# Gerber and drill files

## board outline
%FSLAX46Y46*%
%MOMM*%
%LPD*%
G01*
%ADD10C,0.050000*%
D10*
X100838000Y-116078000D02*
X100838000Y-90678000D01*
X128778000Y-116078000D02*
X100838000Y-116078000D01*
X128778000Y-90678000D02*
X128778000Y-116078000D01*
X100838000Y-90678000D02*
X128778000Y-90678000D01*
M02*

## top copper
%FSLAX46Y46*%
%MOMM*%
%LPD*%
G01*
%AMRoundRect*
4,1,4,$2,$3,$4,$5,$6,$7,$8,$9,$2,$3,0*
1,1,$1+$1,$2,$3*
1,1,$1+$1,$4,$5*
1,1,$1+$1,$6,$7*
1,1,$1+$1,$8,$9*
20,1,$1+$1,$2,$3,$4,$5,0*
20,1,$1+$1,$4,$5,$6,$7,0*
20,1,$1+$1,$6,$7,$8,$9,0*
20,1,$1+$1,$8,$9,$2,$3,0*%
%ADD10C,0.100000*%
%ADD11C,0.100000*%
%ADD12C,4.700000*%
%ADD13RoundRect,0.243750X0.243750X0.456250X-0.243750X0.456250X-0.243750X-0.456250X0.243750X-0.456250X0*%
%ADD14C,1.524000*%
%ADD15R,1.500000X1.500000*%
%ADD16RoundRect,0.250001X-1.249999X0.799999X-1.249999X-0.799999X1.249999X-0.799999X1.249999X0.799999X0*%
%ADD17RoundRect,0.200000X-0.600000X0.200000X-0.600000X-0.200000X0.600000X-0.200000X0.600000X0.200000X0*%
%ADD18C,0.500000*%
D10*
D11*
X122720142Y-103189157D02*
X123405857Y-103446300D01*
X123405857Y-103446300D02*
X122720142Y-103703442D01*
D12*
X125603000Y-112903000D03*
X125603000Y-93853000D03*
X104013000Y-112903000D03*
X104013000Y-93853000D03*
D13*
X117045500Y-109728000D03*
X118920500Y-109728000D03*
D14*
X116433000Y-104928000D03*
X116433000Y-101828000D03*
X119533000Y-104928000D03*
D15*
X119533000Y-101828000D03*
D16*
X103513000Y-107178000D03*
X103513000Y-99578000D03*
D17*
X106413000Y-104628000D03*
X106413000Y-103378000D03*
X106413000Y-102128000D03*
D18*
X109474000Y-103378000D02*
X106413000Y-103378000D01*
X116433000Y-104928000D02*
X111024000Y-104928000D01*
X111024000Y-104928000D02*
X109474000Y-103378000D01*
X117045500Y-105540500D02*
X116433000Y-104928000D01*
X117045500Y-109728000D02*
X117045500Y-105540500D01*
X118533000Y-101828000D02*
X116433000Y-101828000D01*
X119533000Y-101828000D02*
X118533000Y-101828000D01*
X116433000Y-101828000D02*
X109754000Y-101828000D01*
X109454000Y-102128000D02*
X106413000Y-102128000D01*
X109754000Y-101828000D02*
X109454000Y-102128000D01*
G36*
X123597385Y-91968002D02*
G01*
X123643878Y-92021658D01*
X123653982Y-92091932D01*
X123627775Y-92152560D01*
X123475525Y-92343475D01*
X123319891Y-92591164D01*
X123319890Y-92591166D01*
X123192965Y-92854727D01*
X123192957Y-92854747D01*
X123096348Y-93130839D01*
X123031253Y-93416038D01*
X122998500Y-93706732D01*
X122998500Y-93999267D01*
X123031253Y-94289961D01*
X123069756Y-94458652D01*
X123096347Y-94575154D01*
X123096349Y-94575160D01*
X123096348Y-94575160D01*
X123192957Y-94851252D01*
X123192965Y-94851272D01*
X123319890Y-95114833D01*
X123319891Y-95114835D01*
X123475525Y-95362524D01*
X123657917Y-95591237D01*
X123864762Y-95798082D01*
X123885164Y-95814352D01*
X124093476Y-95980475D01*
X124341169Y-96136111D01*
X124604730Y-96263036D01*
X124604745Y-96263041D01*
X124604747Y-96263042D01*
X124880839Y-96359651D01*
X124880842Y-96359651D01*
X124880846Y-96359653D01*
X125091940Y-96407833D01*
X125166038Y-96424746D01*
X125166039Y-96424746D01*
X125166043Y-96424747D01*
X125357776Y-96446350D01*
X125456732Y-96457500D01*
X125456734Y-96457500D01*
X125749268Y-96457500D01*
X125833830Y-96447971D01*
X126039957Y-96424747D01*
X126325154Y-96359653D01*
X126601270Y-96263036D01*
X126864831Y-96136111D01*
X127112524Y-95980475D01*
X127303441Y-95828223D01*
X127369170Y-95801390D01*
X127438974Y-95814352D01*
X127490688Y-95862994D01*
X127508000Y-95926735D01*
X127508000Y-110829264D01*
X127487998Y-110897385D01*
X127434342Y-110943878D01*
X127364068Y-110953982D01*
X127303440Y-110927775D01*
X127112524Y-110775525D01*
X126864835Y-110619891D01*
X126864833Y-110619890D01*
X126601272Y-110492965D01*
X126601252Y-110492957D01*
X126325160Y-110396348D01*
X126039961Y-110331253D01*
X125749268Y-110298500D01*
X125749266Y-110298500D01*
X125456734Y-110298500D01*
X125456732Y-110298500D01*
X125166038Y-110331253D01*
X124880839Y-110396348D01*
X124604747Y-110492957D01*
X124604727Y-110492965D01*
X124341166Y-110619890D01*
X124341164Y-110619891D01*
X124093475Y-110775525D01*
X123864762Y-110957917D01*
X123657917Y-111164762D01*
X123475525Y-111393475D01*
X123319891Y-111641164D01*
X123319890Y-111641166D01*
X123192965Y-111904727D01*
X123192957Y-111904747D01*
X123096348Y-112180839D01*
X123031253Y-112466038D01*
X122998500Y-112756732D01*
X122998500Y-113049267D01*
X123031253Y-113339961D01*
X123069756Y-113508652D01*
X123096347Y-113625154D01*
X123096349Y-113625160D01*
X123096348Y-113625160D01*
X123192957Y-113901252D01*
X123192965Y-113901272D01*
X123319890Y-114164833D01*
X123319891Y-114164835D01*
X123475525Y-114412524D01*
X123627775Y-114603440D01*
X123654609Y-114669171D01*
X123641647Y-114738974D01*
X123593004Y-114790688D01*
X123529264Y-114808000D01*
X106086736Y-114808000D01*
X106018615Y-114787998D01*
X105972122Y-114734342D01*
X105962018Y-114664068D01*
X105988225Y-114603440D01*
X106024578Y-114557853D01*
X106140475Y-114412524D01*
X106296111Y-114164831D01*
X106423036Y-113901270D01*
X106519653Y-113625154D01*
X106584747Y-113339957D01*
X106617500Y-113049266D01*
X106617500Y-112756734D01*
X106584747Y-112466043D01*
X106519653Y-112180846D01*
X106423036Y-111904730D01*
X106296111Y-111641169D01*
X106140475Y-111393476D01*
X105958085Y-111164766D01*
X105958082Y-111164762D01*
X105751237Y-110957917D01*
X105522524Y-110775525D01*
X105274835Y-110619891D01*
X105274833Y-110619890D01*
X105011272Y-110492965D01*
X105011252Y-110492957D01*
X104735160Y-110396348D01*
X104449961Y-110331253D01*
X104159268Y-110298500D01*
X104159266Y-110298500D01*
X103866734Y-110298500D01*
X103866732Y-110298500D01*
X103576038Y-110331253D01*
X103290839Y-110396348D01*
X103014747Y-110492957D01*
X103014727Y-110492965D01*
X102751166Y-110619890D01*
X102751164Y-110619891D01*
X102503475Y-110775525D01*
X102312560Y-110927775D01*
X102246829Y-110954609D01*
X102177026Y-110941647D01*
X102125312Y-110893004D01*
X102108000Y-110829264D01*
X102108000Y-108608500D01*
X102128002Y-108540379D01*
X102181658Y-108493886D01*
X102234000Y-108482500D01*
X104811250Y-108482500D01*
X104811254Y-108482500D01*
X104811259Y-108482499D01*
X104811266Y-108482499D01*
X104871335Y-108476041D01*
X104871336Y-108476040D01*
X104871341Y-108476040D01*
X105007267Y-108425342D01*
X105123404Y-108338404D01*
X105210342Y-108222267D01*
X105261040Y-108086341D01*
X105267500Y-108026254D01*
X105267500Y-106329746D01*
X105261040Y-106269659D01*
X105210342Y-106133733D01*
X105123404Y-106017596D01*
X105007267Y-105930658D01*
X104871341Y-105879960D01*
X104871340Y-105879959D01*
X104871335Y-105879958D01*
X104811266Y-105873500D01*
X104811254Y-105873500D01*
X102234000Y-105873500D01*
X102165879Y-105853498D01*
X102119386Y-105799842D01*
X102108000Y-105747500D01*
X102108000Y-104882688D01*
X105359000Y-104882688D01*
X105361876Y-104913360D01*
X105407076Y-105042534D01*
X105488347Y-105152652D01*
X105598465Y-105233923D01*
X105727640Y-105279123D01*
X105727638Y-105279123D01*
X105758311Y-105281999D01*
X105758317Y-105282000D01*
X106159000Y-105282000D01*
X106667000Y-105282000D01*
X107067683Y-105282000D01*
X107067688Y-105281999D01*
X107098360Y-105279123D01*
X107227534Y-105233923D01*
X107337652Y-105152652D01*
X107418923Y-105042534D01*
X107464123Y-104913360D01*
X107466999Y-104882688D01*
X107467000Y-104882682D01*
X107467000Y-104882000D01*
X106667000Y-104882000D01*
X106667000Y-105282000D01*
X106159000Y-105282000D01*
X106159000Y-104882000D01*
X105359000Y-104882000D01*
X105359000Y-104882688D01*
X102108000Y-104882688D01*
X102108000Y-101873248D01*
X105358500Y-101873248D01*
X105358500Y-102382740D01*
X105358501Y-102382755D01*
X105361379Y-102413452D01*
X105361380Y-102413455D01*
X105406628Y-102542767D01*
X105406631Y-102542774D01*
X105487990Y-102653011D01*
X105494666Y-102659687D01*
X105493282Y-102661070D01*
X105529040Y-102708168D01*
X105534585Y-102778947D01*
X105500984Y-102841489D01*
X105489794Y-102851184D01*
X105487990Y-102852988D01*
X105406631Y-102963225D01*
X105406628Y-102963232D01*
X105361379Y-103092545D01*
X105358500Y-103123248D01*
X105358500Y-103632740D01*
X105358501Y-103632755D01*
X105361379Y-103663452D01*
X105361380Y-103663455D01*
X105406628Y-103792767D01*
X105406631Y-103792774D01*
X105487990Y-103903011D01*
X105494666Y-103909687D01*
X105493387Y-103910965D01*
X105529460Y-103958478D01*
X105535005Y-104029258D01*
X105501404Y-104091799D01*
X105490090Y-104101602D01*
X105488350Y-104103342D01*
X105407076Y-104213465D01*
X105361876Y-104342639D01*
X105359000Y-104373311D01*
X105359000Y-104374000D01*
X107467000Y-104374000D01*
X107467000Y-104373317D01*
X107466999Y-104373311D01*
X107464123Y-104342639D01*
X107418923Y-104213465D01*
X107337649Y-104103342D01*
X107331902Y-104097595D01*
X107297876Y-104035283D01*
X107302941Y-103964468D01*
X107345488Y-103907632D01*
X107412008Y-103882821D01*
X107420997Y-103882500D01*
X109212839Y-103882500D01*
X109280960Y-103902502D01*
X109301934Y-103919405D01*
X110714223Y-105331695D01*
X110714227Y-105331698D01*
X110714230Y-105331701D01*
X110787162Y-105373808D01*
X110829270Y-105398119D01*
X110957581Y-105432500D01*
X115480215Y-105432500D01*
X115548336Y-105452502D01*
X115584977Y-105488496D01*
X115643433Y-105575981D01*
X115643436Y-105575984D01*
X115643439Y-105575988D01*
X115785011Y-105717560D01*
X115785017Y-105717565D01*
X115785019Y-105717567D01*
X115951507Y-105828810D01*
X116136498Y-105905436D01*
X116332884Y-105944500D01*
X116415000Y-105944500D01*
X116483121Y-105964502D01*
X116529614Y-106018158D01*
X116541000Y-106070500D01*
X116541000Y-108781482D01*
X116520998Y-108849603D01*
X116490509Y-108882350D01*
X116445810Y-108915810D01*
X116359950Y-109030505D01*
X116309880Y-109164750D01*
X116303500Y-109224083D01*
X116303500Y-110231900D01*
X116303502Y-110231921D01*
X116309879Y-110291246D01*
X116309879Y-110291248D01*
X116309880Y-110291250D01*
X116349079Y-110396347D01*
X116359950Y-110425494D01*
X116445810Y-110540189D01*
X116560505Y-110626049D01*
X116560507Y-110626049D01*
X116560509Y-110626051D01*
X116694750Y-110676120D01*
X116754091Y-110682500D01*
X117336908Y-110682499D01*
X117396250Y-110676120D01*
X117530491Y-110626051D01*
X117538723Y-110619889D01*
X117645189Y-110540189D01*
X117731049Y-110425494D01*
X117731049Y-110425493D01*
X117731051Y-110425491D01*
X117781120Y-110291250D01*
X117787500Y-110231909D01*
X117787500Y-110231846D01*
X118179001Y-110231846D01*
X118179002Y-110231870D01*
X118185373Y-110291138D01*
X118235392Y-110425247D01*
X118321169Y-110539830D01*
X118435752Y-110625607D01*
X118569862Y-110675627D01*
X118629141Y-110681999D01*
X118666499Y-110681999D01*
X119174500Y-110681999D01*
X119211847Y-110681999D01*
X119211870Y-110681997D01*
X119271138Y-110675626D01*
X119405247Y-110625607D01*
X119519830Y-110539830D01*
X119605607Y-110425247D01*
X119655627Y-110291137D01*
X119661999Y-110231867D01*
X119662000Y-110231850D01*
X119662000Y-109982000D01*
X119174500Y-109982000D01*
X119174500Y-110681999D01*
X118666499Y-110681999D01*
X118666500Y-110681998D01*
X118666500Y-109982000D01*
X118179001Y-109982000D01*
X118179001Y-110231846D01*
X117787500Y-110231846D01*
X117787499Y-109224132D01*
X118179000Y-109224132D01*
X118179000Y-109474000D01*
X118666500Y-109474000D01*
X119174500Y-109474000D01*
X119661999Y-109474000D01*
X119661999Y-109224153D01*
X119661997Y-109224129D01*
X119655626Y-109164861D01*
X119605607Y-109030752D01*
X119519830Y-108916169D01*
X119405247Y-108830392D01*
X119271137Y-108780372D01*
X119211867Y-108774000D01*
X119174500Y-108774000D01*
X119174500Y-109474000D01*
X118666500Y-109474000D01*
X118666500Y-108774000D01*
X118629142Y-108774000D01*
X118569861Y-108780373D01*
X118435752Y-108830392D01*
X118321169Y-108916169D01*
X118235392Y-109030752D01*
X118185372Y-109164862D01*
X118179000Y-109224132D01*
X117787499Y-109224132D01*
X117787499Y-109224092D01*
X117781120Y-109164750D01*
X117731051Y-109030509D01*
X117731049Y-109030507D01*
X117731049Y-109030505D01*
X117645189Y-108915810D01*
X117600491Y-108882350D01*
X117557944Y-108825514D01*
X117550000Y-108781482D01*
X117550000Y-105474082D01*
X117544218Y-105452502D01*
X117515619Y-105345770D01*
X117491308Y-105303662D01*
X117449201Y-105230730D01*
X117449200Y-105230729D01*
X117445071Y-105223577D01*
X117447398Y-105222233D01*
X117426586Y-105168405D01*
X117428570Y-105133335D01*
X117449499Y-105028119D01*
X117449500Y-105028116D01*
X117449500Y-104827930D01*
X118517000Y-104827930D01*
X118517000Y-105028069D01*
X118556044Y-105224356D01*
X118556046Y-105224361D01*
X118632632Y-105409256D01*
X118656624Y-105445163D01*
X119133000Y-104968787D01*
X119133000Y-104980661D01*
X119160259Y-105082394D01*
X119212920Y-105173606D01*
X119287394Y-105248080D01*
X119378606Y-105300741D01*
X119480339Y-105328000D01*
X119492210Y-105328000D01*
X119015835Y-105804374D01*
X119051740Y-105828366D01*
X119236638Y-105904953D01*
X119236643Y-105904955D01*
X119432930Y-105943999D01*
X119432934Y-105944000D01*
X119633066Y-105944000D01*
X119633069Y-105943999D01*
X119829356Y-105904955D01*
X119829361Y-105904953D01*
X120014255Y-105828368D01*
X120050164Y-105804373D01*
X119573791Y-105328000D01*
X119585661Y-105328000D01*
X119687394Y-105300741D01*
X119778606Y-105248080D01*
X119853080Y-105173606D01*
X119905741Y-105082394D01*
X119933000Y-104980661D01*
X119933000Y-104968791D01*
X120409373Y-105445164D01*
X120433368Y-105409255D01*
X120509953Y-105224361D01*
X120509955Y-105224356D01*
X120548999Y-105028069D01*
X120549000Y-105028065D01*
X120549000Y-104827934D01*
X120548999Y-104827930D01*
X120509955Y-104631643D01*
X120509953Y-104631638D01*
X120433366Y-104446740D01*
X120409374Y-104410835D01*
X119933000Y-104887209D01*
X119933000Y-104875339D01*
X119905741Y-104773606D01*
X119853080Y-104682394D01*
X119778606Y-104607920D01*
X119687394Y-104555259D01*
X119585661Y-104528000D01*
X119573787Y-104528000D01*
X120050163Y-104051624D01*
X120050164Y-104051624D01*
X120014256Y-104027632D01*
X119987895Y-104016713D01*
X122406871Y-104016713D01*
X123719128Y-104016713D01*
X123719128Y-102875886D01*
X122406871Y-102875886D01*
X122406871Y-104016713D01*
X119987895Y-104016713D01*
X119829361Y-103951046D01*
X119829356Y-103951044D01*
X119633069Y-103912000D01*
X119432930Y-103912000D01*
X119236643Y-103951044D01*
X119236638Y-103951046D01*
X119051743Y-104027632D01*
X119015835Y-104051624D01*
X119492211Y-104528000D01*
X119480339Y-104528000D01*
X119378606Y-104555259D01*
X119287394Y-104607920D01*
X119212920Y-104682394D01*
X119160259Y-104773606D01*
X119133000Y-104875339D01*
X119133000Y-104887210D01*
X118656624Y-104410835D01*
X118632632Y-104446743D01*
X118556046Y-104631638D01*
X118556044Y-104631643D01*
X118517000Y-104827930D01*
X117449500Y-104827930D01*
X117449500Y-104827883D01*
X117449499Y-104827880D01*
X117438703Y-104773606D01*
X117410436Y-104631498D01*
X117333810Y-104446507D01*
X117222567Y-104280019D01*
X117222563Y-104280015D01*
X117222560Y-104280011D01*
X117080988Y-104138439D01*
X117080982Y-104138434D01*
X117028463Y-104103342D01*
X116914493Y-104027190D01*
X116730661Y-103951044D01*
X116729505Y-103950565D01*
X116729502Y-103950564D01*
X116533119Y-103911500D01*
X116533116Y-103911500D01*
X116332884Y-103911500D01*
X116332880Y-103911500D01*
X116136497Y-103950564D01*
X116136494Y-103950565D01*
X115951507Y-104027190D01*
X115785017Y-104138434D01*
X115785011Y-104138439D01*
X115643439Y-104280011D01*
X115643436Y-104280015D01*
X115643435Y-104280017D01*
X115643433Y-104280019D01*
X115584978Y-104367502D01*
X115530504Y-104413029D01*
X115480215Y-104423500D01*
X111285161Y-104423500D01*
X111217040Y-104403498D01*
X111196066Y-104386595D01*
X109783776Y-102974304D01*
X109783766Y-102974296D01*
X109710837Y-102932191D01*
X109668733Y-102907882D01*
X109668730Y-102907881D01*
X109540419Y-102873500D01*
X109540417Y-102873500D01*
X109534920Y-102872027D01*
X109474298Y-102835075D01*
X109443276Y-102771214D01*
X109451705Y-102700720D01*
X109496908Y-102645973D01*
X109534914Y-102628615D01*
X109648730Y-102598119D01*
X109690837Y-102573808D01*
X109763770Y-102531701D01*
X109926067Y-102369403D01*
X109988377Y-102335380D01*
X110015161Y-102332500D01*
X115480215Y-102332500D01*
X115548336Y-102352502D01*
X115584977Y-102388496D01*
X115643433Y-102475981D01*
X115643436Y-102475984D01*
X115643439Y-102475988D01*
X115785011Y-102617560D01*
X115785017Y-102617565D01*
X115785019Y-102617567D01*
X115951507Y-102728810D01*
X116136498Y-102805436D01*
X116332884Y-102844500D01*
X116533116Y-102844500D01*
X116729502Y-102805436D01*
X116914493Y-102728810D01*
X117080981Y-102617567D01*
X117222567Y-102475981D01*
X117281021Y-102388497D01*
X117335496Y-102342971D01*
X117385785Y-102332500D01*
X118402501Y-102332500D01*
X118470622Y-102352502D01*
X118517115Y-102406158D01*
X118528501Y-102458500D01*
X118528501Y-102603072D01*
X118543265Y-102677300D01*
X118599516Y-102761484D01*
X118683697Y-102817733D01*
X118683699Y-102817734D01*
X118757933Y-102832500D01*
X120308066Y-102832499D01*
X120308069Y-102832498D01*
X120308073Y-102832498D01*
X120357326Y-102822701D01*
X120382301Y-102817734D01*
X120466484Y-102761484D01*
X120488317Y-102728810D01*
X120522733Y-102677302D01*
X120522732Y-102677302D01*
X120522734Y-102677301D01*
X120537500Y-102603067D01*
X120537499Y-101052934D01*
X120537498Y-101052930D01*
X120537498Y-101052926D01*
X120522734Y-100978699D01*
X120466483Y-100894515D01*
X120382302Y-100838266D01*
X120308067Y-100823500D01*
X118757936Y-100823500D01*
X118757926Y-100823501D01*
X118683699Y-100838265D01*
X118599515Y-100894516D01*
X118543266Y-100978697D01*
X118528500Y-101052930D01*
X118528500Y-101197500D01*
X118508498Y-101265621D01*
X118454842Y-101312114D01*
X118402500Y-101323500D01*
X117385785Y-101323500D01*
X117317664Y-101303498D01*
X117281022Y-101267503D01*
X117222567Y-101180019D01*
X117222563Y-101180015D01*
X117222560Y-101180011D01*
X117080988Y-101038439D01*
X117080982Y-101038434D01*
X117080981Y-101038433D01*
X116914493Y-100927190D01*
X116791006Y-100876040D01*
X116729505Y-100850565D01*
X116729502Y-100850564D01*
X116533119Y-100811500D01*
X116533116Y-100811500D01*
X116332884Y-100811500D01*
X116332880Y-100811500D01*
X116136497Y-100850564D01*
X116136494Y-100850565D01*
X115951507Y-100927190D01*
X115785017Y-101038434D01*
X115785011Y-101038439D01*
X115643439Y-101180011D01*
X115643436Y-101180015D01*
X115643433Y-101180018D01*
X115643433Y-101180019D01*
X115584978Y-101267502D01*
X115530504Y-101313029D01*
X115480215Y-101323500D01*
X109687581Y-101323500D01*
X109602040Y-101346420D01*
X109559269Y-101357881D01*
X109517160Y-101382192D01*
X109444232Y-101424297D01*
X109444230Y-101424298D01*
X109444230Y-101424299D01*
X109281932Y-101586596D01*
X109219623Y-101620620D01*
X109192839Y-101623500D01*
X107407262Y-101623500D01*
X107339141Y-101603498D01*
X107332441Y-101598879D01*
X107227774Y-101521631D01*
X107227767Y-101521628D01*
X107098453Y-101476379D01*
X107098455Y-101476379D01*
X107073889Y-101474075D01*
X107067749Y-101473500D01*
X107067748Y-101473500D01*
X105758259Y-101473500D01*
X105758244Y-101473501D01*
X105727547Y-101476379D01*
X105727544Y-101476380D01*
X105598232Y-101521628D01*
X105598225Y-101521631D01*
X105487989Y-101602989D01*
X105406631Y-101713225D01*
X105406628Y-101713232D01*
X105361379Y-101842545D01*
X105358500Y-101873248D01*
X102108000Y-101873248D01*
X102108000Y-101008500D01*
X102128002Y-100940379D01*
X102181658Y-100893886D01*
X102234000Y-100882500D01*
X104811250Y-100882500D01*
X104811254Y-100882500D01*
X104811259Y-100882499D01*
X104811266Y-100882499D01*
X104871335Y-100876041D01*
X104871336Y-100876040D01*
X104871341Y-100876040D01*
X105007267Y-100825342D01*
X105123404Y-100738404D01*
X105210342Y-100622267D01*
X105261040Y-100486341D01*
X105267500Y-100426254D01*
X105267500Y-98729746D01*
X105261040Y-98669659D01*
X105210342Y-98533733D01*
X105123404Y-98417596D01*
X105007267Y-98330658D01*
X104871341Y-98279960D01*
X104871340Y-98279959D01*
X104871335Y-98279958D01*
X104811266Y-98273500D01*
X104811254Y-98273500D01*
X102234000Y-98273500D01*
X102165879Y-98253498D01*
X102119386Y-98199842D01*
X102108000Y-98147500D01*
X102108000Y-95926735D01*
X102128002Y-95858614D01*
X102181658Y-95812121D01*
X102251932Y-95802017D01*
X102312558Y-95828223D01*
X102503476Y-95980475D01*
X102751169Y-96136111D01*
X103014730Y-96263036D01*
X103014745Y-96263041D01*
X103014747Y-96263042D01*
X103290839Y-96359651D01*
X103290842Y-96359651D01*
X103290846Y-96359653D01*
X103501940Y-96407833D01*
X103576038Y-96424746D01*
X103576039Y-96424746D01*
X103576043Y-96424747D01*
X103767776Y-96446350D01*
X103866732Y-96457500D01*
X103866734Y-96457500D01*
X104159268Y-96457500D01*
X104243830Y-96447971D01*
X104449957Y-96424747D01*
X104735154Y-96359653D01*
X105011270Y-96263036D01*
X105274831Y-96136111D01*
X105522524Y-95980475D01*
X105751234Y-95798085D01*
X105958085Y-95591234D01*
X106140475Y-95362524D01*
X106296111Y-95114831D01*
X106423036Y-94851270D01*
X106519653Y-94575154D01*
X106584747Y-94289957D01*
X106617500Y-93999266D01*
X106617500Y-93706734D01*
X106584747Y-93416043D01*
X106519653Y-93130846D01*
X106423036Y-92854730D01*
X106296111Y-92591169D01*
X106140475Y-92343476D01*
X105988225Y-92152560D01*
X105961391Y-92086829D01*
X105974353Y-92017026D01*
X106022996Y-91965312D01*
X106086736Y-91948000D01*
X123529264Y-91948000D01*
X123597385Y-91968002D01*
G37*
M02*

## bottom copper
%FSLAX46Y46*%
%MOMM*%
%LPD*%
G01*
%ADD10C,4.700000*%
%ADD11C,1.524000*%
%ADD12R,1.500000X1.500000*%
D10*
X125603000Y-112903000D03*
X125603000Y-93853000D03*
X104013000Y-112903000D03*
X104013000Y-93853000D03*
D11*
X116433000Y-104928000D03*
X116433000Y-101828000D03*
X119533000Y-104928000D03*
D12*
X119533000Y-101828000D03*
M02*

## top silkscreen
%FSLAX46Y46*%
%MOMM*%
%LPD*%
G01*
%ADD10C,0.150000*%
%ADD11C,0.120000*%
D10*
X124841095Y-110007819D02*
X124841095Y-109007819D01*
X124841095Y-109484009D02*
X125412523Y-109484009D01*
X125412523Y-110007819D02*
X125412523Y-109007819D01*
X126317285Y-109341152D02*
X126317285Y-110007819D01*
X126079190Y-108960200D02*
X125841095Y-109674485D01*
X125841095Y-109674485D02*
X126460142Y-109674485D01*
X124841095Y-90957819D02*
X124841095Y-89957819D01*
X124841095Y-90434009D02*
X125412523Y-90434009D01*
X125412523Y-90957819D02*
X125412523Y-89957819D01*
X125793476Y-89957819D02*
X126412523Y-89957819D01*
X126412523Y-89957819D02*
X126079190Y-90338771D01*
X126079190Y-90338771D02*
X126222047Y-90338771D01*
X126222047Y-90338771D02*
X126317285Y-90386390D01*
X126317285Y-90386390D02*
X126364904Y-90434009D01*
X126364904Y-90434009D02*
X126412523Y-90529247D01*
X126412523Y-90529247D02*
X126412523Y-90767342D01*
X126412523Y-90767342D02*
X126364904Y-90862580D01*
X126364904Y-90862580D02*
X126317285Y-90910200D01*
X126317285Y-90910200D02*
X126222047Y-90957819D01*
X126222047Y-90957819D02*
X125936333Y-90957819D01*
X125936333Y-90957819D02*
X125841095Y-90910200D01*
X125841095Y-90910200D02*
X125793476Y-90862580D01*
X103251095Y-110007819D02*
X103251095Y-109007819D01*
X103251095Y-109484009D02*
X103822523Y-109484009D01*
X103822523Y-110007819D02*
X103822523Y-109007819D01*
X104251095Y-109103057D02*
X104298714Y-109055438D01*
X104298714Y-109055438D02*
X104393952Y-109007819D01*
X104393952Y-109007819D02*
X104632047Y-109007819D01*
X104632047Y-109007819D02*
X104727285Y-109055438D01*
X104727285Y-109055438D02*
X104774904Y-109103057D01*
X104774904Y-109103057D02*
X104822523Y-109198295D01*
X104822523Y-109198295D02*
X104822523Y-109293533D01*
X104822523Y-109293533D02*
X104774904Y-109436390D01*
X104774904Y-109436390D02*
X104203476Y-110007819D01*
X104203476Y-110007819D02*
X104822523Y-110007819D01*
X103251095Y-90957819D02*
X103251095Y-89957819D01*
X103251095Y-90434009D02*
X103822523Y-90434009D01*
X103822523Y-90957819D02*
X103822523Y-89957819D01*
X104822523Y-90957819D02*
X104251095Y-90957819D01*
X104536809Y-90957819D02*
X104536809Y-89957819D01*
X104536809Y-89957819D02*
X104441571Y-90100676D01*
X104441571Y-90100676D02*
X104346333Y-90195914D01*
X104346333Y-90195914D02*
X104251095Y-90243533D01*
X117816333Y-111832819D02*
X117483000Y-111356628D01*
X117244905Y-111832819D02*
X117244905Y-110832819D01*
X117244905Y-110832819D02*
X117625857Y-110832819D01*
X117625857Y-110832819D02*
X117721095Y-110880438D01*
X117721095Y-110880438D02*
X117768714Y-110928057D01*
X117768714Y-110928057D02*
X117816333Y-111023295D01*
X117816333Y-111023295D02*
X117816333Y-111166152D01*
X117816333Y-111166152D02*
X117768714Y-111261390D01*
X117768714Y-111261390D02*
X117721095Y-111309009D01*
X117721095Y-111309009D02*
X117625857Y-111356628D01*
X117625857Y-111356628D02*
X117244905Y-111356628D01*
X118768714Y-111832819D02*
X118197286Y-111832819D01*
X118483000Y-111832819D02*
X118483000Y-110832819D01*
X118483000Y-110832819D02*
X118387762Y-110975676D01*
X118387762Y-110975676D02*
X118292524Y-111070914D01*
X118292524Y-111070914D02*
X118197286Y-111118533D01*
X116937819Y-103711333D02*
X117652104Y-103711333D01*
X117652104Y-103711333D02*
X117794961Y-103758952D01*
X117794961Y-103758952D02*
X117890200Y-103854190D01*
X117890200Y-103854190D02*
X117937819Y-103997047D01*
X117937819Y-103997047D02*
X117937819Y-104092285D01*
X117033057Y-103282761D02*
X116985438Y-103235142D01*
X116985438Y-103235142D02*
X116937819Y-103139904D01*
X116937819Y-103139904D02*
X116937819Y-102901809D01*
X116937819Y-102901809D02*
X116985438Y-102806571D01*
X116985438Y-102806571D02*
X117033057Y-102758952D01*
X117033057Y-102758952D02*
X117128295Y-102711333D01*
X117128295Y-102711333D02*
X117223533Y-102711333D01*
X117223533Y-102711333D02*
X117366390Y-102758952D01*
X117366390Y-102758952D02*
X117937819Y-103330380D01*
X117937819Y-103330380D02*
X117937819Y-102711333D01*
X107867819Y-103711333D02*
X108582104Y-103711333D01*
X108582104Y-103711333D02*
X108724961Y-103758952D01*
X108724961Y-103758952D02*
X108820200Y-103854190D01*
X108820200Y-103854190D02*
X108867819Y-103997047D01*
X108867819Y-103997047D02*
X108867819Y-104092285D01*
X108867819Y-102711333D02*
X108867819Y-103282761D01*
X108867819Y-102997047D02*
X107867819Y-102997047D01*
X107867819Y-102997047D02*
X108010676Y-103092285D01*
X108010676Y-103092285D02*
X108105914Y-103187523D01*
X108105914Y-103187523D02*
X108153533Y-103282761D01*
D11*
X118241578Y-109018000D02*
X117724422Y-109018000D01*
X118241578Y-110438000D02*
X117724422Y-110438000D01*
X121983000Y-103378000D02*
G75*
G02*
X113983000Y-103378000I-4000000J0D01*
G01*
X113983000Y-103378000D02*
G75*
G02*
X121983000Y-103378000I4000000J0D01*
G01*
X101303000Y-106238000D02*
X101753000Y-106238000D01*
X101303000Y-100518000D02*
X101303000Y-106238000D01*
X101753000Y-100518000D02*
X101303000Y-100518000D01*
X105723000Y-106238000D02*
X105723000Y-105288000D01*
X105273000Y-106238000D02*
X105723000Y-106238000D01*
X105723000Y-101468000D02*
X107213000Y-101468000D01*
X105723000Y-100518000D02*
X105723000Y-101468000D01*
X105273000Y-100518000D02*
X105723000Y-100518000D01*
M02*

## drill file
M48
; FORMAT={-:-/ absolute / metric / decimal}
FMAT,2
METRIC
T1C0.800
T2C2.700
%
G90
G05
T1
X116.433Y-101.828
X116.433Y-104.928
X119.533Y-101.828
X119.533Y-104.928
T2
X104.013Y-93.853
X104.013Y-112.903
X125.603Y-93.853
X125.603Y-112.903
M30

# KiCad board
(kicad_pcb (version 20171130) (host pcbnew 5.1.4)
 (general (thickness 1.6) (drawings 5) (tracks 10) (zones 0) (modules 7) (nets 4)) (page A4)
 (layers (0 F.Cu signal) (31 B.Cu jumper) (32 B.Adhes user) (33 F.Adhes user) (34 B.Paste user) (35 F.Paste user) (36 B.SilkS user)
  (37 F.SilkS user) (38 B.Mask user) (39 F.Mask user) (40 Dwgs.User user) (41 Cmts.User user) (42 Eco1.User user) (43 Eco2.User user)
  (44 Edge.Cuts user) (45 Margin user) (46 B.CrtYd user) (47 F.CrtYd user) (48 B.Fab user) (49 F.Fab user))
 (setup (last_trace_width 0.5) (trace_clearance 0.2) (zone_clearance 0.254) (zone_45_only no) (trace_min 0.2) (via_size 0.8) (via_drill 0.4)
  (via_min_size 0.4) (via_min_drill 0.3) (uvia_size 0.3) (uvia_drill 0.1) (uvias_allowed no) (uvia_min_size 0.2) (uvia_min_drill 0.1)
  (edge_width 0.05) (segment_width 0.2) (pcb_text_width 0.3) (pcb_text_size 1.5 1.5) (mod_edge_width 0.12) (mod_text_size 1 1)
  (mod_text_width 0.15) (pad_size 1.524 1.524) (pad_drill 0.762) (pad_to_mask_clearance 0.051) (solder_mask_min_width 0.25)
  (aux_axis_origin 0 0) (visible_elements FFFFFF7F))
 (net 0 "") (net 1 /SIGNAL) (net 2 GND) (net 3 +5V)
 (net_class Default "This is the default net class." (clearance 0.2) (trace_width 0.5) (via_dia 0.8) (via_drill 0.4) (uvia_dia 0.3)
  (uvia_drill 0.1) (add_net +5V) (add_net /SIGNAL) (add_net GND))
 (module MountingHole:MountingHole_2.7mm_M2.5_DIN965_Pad (layer F.Cu) (at 125.603 112.903)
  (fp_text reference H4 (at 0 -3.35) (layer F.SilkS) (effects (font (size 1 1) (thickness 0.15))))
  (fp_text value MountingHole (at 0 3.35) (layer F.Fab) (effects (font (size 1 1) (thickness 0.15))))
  (pad 1 thru_hole circle (at 0 0) (size 4.7 4.7) (drill 2.7) (layers *.Cu *.Mask)))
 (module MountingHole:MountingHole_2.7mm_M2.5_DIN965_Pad (layer F.Cu) (at 125.603 93.853)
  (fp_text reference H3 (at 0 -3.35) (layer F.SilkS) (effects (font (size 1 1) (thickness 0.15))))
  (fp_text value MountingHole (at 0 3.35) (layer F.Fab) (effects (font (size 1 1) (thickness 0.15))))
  (pad 1 thru_hole circle (at 0 0) (size 4.7 4.7) (drill 2.7) (layers *.Cu *.Mask)))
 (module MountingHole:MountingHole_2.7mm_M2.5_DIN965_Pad (layer F.Cu) (at 104.013 112.903)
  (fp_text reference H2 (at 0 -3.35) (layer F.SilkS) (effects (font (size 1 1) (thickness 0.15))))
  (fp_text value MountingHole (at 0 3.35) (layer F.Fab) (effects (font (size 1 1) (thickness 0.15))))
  (pad 1 thru_hole circle (at 0 0) (size 4.7 4.7) (drill 2.7) (layers *.Cu *.Mask)))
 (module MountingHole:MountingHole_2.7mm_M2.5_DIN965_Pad (layer F.Cu) (at 104.013 93.853)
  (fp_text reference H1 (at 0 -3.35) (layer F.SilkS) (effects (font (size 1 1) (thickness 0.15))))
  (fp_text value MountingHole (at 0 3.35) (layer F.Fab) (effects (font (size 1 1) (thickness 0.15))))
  (pad 1 thru_hole circle (at 0 0) (size 4.7 4.7) (drill 2.7) (layers *.Cu *.Mask)))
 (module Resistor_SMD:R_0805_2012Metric (layer F.Cu) (at 117.983 109.728 180)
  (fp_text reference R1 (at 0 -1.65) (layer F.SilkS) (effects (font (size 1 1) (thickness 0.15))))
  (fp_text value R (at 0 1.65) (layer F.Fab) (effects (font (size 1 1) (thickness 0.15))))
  (fp_line (start -0.258578 0.71) (end 0.258578 0.71) (layer F.SilkS) (width 0.12))
  (fp_line (start -0.258578 -0.71) (end 0.258578 -0.71) (layer F.SilkS) (width 0.12))
  (pad 2 smd roundrect (at 0.9375 0 180) (size 0.975 1.4) (layers F.Cu F.Paste F.Mask) (roundrect_rratio 0.25) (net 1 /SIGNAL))
  (pad 1 smd roundrect (at -0.9375 0 180) (size 0.975 1.4) (layers F.Cu F.Paste F.Mask) (roundrect_rratio 0.25) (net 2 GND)))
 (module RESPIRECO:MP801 (layer F.Cu) (at 117.983 103.378 270)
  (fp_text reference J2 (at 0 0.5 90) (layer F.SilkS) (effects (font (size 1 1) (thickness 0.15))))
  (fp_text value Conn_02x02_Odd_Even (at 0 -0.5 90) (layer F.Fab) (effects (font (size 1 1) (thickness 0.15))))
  (fp_circle (center 0 0) (end 4 0) (layer F.SilkS) (width 0.12))
  (pad 4 thru_hole circle (at 1.55 1.55 270) (size 1.524 1.524) (drill 0.8) (layers *.Cu *.Mask) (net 1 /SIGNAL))
  (pad 3 thru_hole circle (at -1.55 1.55 270) (size 1.524 1.524) (drill 0.8) (layers *.Cu *.Mask) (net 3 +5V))
  (pad 2 thru_hole circle (at 1.55 -1.55 270) (size 1.524 1.524) (drill 0.8) (layers *.Cu *.Mask) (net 2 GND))
  (pad 1 thru_hole rect (at -1.55 -1.55 270) (size 1.5 1.5) (drill 0.8) (layers *.Cu *.Mask) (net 3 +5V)))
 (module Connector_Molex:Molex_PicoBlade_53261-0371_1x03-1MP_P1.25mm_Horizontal (layer F.Cu) (at 104.013 103.378 270)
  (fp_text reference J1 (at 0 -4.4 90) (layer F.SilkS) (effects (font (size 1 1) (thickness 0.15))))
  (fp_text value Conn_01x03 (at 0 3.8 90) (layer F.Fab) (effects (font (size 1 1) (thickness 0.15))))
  (fp_line (start 2.86 2.71) (end 2.86 2.26) (layer F.SilkS) (width 0.12))
  (fp_line (start -2.86 2.71) (end 2.86 2.71) (layer F.SilkS) (width 0.12))
  (fp_line (start -2.86 2.26) (end -2.86 2.71) (layer F.SilkS) (width 0.12))
  (fp_line (start 2.86 -1.71) (end 1.91 -1.71) (layer F.SilkS) (width 0.12))
  (fp_line (start 2.86 -1.26) (end 2.86 -1.71) (layer F.SilkS) (width 0.12))
  (fp_line (start -1.91 -1.71) (end -1.91 -3.2) (layer F.SilkS) (width 0.12))
  (fp_line (start -2.86 -1.71) (end -1.91 -1.71) (layer F.SilkS) (width 0.12))
  (fp_line (start -2.86 -1.26) (end -2.86 -1.71) (layer F.SilkS) (width 0.12))
  (pad MP smd roundrect (at 3.8 0.5 270) (size 2.1 3) (layers F.Cu F.Paste F.Mask) (roundrect_rratio 0.119048))
  (pad MP smd roundrect (at -3.8 0.5 270) (size 2.1 3) (layers F.Cu F.Paste F.Mask) (roundrect_rratio 0.119048))
  (pad 3 smd roundrect (at 1.25 -2.4 270) (size 0.8 1.6) (layers F.Cu F.Paste F.Mask) (roundrect_rratio 0.25) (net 2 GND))
  (pad 2 smd roundrect (at 0 -2.4 270) (size 0.8 1.6) (layers F.Cu F.Paste F.Mask) (roundrect_rratio 0.25) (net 1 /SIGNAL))
  (pad 1 smd roundrect (at -1.25 -2.4 270) (size 0.8 1.6) (layers F.Cu F.Paste F.Mask) (roundrect_rratio 0.25) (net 3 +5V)))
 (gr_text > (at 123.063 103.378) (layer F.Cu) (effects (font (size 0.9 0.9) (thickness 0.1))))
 (gr_line (start 100.838 116.078) (end 100.838 90.678) (layer Edge.Cuts) (width 0.05))
 (gr_line (start 128.778 116.078) (end 100.838 116.078) (layer Edge.Cuts) (width 0.05))
 (gr_line (start 128.778 90.678) (end 128.778 116.078) (layer Edge.Cuts) (width 0.05))
 (gr_line (start 100.838 90.678) (end 128.778 90.678) (layer Edge.Cuts) (width 0.05))
 (segment (start 109.474 103.378) (end 106.413 103.378) (width 0.5) (layer F.Cu) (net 1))
 (segment (start 116.433 104.928) (end 111.024 104.928) (width 0.5) (layer F.Cu) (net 1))
 (segment (start 111.024 104.928) (end 109.474 103.378) (width 0.5) (layer F.Cu) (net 1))
 (segment (start 117.0455 105.5405) (end 116.433 104.928) (width 0.5) (layer F.Cu) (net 1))
 (segment (start 117.0455 109.728) (end 117.0455 105.5405) (width 0.5) (layer F.Cu) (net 1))
 (segment (start 118.533 101.828) (end 116.433 101.828) (width 0.5) (layer F.Cu) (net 3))
 (segment (start 119.533 101.828) (end 118.533 101.828) (width 0.5) (layer F.Cu) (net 3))
 (segment (start 116.433 101.828) (end 109.754 101.828) (width 0.5) (layer F.Cu) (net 3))
 (segment (start 109.454 102.128) (end 106.413 102.128) (width 0.5) (layer F.Cu) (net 3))
 (segment (start 109.754 101.828) (end 109.454 102.128) (width 0.5) (layer F.Cu) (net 3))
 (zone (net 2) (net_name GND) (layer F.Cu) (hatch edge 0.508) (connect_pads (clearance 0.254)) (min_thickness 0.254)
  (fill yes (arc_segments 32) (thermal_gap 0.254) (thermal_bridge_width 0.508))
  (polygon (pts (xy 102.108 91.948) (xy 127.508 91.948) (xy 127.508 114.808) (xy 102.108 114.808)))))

